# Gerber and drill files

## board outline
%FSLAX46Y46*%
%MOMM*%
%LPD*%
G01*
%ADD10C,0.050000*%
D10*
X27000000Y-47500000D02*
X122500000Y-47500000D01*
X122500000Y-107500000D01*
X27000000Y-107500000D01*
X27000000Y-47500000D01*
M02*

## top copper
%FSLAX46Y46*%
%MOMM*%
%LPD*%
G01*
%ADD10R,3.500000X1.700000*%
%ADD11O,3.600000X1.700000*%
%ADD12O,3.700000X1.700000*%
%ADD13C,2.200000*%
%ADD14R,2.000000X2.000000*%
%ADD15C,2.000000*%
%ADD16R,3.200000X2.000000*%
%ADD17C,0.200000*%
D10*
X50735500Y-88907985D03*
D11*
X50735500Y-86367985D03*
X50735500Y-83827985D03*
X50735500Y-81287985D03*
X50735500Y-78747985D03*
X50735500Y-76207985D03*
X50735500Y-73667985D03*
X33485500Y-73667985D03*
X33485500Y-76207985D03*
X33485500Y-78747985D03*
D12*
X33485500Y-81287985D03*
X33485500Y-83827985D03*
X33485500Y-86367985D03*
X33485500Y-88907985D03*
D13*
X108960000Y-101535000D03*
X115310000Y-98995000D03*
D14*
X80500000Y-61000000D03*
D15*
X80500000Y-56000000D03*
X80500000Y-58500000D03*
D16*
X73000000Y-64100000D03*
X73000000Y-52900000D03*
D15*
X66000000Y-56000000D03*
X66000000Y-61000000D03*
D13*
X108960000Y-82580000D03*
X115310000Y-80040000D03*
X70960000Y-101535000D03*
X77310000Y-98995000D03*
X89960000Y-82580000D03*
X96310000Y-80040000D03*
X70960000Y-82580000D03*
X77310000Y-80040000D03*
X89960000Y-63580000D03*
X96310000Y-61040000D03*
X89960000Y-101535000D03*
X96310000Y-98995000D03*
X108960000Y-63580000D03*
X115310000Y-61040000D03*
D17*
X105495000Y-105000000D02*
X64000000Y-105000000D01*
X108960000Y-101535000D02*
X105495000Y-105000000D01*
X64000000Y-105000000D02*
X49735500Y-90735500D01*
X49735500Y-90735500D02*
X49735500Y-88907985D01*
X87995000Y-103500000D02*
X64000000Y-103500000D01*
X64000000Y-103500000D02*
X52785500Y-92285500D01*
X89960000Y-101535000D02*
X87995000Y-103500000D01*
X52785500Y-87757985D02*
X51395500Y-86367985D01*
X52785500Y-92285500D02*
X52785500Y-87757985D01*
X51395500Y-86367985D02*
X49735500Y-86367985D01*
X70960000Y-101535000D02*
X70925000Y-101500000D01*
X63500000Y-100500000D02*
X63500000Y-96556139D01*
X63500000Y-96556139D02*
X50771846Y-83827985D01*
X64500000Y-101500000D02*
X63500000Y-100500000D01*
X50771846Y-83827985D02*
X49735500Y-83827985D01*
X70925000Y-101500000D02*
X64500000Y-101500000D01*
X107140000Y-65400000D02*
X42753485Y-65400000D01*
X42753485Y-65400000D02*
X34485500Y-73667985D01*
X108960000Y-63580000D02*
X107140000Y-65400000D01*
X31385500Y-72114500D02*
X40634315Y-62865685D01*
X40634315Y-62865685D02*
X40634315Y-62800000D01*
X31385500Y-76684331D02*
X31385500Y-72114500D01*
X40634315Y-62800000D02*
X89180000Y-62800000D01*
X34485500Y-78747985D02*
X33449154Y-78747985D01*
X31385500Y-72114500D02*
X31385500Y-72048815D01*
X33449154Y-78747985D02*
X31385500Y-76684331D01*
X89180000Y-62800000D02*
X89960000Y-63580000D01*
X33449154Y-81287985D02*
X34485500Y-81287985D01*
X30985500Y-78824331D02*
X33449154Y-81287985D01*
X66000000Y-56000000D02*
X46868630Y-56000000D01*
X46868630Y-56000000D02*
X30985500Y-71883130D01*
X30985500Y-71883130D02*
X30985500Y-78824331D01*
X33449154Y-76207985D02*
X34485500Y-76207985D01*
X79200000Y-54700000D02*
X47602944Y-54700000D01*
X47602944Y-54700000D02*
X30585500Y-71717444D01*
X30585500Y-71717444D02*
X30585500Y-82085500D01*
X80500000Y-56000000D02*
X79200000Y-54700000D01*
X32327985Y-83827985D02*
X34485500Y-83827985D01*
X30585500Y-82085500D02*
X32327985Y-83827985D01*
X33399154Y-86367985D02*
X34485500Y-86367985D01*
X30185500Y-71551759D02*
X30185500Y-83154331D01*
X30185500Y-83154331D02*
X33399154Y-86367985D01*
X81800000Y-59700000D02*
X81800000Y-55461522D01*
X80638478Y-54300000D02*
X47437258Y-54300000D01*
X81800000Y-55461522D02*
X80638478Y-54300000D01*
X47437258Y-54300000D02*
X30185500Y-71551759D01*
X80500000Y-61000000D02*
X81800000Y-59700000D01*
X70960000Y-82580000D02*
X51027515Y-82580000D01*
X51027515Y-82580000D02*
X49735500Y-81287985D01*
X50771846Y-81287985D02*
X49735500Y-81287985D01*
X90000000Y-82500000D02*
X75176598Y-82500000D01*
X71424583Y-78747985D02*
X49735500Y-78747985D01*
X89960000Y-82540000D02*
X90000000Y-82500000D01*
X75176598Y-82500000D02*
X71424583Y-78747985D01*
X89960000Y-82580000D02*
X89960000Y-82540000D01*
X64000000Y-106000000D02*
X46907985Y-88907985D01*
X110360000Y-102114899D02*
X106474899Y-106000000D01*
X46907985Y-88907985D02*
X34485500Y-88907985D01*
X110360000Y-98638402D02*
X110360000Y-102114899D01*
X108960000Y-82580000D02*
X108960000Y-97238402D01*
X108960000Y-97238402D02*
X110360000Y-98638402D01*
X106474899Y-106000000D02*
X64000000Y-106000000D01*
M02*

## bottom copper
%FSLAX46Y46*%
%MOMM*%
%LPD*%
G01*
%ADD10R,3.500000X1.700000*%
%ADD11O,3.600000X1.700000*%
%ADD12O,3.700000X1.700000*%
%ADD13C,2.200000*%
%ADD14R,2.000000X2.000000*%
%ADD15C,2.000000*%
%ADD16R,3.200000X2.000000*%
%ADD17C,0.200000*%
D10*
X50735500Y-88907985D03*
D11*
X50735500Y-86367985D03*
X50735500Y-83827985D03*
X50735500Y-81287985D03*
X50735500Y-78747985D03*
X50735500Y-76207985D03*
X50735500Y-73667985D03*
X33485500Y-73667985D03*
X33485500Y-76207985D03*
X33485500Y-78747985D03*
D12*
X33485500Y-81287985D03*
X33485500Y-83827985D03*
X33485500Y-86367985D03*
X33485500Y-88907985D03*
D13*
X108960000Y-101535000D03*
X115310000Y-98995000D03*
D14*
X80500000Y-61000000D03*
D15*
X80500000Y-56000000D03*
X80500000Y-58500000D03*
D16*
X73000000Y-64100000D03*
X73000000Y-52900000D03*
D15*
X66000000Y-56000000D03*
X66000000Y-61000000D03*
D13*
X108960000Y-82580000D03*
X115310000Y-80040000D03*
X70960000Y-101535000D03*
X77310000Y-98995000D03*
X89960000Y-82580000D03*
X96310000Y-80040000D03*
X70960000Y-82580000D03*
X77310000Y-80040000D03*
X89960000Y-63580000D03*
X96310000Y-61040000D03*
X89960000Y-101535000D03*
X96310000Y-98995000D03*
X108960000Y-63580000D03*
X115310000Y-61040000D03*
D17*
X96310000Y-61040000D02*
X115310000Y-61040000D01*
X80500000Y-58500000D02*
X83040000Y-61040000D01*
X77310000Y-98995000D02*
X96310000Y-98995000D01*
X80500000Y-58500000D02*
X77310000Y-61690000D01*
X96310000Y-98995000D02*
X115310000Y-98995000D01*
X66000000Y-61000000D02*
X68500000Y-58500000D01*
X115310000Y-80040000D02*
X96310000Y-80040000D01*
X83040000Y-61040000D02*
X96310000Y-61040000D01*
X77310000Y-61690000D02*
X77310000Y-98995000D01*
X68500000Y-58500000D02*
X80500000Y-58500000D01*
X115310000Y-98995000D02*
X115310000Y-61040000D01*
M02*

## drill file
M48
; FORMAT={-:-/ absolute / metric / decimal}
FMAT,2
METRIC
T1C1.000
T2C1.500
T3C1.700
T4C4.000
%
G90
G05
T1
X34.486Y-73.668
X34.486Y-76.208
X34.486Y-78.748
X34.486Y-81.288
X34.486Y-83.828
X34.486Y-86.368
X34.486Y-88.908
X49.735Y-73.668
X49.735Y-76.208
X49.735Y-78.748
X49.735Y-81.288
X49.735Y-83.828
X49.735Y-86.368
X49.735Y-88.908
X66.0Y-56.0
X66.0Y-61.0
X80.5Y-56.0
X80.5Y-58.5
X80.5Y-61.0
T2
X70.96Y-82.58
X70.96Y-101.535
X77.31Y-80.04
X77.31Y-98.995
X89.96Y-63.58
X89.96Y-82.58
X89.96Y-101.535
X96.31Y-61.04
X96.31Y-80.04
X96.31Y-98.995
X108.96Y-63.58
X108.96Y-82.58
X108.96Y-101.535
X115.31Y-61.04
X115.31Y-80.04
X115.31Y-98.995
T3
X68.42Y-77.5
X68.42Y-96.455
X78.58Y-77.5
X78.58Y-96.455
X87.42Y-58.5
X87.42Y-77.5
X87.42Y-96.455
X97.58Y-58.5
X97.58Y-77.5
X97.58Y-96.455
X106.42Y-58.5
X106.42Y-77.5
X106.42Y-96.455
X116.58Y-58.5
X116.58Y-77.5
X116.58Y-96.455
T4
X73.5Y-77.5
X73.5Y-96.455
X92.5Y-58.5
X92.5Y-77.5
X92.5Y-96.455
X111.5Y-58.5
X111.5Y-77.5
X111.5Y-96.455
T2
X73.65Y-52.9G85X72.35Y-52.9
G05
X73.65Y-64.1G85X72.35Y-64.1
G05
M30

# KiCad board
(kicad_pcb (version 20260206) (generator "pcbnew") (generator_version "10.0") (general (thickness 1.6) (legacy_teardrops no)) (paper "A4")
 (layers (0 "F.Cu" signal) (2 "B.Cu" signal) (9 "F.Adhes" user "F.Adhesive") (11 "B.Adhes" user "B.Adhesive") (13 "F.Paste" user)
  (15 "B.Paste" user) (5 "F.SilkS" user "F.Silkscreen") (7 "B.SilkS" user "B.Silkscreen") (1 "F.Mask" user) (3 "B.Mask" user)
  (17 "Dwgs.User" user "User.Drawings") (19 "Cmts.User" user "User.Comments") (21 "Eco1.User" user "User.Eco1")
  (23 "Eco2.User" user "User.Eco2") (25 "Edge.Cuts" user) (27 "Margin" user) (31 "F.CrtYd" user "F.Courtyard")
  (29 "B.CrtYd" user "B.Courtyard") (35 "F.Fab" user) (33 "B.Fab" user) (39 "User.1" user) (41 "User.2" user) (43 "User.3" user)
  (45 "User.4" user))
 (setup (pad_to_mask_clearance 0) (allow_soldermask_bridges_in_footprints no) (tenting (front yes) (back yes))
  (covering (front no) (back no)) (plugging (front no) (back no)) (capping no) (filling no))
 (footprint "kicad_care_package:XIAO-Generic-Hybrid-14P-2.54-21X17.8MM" (layer "F.Cu") (at 42.1105 81.287985 180)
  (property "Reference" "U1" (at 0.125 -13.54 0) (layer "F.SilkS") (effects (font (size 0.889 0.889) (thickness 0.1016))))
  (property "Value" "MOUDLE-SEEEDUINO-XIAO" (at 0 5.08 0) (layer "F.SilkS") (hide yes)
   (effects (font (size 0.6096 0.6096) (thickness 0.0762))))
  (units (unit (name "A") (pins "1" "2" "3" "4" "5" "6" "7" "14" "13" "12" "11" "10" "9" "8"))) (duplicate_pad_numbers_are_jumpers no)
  (pad "1" thru_hole rect (at -7.625 -7.62 180) (size 3.5 1.7) (drill 1 (offset -1 0)) (layers "*.Cu" "*.Mask") (remove_unused_layers no)
   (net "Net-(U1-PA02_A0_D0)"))
  (pad "2" thru_hole oval (at -7.625 -5.08 180) (size 3.6 1.7) (drill 1 (offset -1 0)) (layers "*.Cu" "*.Mask") (remove_unused_layers no)
   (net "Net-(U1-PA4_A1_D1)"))
  (pad "3" thru_hole oval (at -7.625 -2.54 180) (size 3.6 1.7) (drill 1 (offset -1 0)) (layers "*.Cu" "*.Mask") (remove_unused_layers no)
   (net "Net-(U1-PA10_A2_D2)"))
  (pad "4" thru_hole oval (at -7.625 0 180) (size 3.6 1.7) (drill 1 (offset -1 0)) (layers "*.Cu" "*.Mask") (remove_unused_layers no)
   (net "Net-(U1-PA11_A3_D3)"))
  (pad "5" thru_hole oval (at -7.625 2.54 180) (size 3.6 1.7) (drill 1 (offset -1 0)) (layers "*.Cu" "*.Mask") (remove_unused_layers no)
   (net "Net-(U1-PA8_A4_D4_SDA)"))
  (pad "6" thru_hole oval (at -7.625 5.08) (size 3.6 1.7) (drill 1 (offset 1 0)) (layers "*.Cu" "*.Mask") (remove_unused_layers no)
   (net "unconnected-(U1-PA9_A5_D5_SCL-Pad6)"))
  (pad "7" thru_hole oval (at -7.625 7.62 180) (size 3.6 1.7) (drill 1 (offset -1 0)) (layers "*.Cu" "*.Mask") (remove_unused_layers no)
   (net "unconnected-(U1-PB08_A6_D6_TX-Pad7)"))
  (pad "8" thru_hole oval (at 7.625 7.62 180) (size 3.6 1.7) (drill 1 (offset 1 0)) (layers "*.Cu" "*.Mask") (remove_unused_layers no)
   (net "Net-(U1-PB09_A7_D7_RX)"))
  (pad "9" thru_hole oval (at 7.625 5.08 180) (size 3.6 1.7) (drill 1 (offset 1 0)) (layers "*.Cu" "*.Mask") (remove_unused_layers no)
   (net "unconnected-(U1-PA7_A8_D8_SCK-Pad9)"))
  (pad "10" thru_hole oval (at 7.625 2.54 180) (size 3.6 1.7) (drill 1 (offset 1 0)) (layers "*.Cu" "*.Mask") (remove_unused_layers no)
   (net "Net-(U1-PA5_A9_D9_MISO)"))
  (pad "11" thru_hole oval (at 7.625 0 180) (size 3.7 1.7) (drill 1 (offset 1 0)) (layers "*.Cu" "*.Mask") (remove_unused_layers no)
   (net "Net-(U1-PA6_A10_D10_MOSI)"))
  (pad "12" thru_hole oval (at 7.625 -2.54 180) (size 3.7 1.7) (drill 1 (offset 1 0)) (layers "*.Cu" "*.Mask") (remove_unused_layers no)
   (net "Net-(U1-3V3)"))
  (pad "13" thru_hole oval (at 7.625 -5.08 180) (size 3.7 1.7) (drill 1 (offset 1 0)) (layers "*.Cu" "*.Mask") (remove_unused_layers no)
   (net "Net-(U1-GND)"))
  (pad "14" thru_hole oval (at 7.625 -7.62 180) (size 3.7 1.7) (drill 1 (offset 1 0)) (layers "*.Cu" "*.Mask") (remove_unused_layers no)
   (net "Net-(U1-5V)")))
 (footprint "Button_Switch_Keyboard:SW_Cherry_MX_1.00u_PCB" (layer "F.Cu") (at 108.96 101.535 180)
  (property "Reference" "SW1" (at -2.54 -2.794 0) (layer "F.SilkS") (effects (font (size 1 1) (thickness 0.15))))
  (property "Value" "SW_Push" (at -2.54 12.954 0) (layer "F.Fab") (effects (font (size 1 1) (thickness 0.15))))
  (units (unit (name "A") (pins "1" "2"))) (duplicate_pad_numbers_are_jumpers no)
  (pad "" np_thru_hole circle (at -7.62 5.08 180) (size 1.7 1.7) (drill 1.7) (layers "*.Cu" "*.Mask"))
  (pad "" np_thru_hole circle (at -2.54 5.08 180) (size 4 4) (drill 4) (layers "*.Cu" "*.Mask"))
  (pad "" np_thru_hole circle (at 2.54 5.08 180) (size 1.7 1.7) (drill 1.7) (layers "*.Cu" "*.Mask"))
  (pad "1" thru_hole circle (at 0 0 180) (size 2.2 2.2) (drill 1.5) (layers "*.Cu" "*.Mask") (remove_unused_layers no)
   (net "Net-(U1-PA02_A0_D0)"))
  (pad "2" thru_hole circle (at -6.35 2.54 180) (size 2.2 2.2) (drill 1.5) (layers "*.Cu" "*.Mask") (remove_unused_layers no) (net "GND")))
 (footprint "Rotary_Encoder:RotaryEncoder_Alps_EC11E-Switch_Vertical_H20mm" (layer "F.Cu") (at 80.5 61 180)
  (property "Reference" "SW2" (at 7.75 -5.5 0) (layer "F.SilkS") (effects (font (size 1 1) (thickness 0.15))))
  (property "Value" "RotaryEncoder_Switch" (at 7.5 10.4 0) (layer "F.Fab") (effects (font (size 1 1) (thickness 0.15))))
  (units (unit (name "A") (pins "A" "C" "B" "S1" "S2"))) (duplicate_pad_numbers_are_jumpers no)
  (pad "A" thru_hole rect (at 0 0 180) (size 2 2) (drill 1) (layers "*.Cu" "*.Mask") (remove_unused_layers no) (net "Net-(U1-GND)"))
  (pad "B" thru_hole circle (at 0 5 180) (size 2 2) (drill 1) (layers "*.Cu" "F.Mask") (remove_unused_layers no) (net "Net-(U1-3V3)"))
  (pad "C" thru_hole circle (at 0 2.5 180) (size 2 2) (drill 1) (layers "*.Cu" "*.Mask") (remove_unused_layers no) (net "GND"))
  (pad "MP" thru_hole rect (at 7.5 -3.1 180) (size 3.2 2) (drill oval 2.8 1.5) (layers "*.Cu" "*.Mask") (remove_unused_layers no))
  (pad "MP" thru_hole rect (at 7.5 8.1 180) (size 3.2 2) (drill oval 2.8 1.5) (layers "*.Cu" "*.Mask") (remove_unused_layers no))
  (pad "S1" thru_hole circle (at 14.5 5 180) (size 2 2) (drill 1) (layers "*.Cu" "*.Mask") (remove_unused_layers no)
   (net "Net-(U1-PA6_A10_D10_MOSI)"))
  (pad "S2" thru_hole circle (at 14.5 0 180) (size 2 2) (drill 1) (layers "*.Cu" "*.Mask") (remove_unused_layers no) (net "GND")))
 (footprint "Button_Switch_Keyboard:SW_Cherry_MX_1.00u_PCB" (layer "F.Cu") (at 108.96 82.58 180)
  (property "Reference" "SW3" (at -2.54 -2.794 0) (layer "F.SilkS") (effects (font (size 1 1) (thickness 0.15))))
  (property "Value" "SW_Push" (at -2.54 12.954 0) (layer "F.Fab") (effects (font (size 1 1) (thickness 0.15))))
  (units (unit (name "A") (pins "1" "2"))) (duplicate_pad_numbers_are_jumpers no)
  (pad "" np_thru_hole circle (at -7.62 5.08 180) (size 1.7 1.7) (drill 1.7) (layers "*.Cu" "*.Mask"))
  (pad "" np_thru_hole circle (at -2.54 5.08 180) (size 4 4) (drill 4) (layers "*.Cu" "*.Mask"))
  (pad "" np_thru_hole circle (at 2.54 5.08 180) (size 1.7 1.7) (drill 1.7) (layers "*.Cu" "*.Mask"))
  (pad "1" thru_hole circle (at 0 0 180) (size 2.2 2.2) (drill 1.5) (layers "*.Cu" "*.Mask") (remove_unused_layers no) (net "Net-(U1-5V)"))
  (pad "2" thru_hole circle (at -6.35 2.54 180) (size 2.2 2.2) (drill 1.5) (layers "*.Cu" "*.Mask") (remove_unused_layers no) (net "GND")))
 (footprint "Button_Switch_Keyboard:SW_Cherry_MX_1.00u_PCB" (layer "F.Cu") (at 70.96 101.535 180)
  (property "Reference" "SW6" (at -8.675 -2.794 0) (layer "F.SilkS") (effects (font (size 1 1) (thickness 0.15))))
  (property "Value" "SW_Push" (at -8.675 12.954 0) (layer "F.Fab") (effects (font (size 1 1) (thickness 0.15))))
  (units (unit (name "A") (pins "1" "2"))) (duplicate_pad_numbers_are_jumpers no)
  (pad "" np_thru_hole circle (at -7.62 5.08 180) (size 1.7 1.7) (drill 1.7) (layers "*.Cu" "*.Mask"))
  (pad "" np_thru_hole circle (at -2.54 5.08 180) (size 4 4) (drill 4) (layers "*.Cu" "*.Mask"))
  (pad "" np_thru_hole circle (at 2.54 5.08 180) (size 1.7 1.7) (drill 1.7) (layers "*.Cu" "*.Mask"))
  (pad "1" thru_hole circle (at 0 0 180) (size 2.2 2.2) (drill 1.5) (layers "*.Cu" "*.Mask") (remove_unused_layers no)
   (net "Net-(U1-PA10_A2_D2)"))
  (pad "2" thru_hole circle (at -6.35 2.54 180) (size 2.2 2.2) (drill 1.5) (layers "*.Cu" "*.Mask") (remove_unused_layers no) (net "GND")))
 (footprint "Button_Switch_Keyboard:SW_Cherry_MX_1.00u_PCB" (layer "F.Cu") (at 89.96 82.58 180)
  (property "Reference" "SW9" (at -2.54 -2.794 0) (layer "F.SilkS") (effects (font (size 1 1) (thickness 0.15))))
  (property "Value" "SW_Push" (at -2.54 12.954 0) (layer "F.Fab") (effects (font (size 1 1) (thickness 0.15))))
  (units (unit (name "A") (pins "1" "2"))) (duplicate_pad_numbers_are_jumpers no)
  (pad "" np_thru_hole circle (at -7.62 5.08 180) (size 1.7 1.7) (drill 1.7) (layers "*.Cu" "*.Mask"))
  (pad "" np_thru_hole circle (at -2.54 5.08 180) (size 4 4) (drill 4) (layers "*.Cu" "*.Mask"))
  (pad "" np_thru_hole circle (at 2.54 5.08 180) (size 1.7 1.7) (drill 1.7) (layers "*.Cu" "*.Mask"))
  (pad "1" thru_hole circle (at 0 0 180) (size 2.2 2.2) (drill 1.5) (layers "*.Cu" "*.Mask") (remove_unused_layers no)
   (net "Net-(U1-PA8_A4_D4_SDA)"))
  (pad "2" thru_hole circle (at -6.35 2.54 180) (size 2.2 2.2) (drill 1.5) (layers "*.Cu" "*.Mask") (remove_unused_layers no) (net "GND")))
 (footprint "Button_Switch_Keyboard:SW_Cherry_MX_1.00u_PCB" (layer "F.Cu") (at 70.96 82.58 180)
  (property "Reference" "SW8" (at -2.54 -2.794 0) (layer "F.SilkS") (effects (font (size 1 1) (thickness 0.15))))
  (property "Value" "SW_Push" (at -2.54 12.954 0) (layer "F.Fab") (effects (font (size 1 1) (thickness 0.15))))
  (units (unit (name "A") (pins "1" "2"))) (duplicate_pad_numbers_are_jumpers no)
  (pad "" np_thru_hole circle (at -7.62 5.08 180) (size 1.7 1.7) (drill 1.7) (layers "*.Cu" "*.Mask"))
  (pad "" np_thru_hole circle (at -2.54 5.08 180) (size 4 4) (drill 4) (layers "*.Cu" "*.Mask"))
  (pad "" np_thru_hole circle (at 2.54 5.08 180) (size 1.7 1.7) (drill 1.7) (layers "*.Cu" "*.Mask"))
  (pad "1" thru_hole circle (at 0 0 180) (size 2.2 2.2) (drill 1.5) (layers "*.Cu" "*.Mask") (remove_unused_layers no)
   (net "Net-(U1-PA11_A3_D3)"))
  (pad "2" thru_hole circle (at -6.35 2.54 180) (size 2.2 2.2) (drill 1.5) (layers "*.Cu" "*.Mask") (remove_unused_layers no) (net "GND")))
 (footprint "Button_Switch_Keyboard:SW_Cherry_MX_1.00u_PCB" (layer "F.Cu") (at 89.96 63.58 180)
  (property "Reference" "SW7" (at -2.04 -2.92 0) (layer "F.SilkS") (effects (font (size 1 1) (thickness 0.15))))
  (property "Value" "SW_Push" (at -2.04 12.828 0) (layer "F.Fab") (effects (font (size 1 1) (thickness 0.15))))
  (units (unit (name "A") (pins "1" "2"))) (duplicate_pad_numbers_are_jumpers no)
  (pad "" np_thru_hole circle (at -7.62 5.08 180) (size 1.7 1.7) (drill 1.7) (layers "*.Cu" "*.Mask"))
  (pad "" np_thru_hole circle (at -2.54 5.08 180) (size 4 4) (drill 4) (layers "*.Cu" "*.Mask"))
  (pad "" np_thru_hole circle (at 2.54 5.08 180) (size 1.7 1.7) (drill 1.7) (layers "*.Cu" "*.Mask"))
  (pad "1" thru_hole circle (at 0 0 180) (size 2.2 2.2) (drill 1.5) (layers "*.Cu" "*.Mask") (remove_unused_layers no)
   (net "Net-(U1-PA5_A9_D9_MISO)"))
  (pad "2" thru_hole circle (at -6.35 2.54 180) (size 2.2 2.2) (drill 1.5) (layers "*.Cu" "*.Mask") (remove_unused_layers no) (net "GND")))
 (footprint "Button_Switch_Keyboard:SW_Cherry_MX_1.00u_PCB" (layer "F.Cu") (at 89.96 101.535 180)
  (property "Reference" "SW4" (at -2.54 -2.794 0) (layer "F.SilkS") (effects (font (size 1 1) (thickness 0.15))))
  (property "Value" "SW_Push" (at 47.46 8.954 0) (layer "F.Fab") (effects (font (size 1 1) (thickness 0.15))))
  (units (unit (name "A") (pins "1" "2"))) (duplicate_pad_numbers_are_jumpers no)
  (pad "" np_thru_hole circle (at -7.62 5.08 180) (size 1.7 1.7) (drill 1.7) (layers "*.Cu" "*.Mask"))
  (pad "" np_thru_hole circle (at -2.54 5.08 180) (size 4 4) (drill 4) (layers "*.Cu" "*.Mask"))
  (pad "" np_thru_hole circle (at 2.54 5.08 180) (size 1.7 1.7) (drill 1.7) (layers "*.Cu" "*.Mask"))
  (pad "1" thru_hole circle (at 0 0 180) (size 2.2 2.2) (drill 1.5) (layers "*.Cu" "*.Mask") (remove_unused_layers no)
   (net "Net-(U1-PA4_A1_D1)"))
  (pad "2" thru_hole circle (at -6.35 2.54 180) (size 2.2 2.2) (drill 1.5) (layers "*.Cu" "*.Mask") (remove_unused_layers no) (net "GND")))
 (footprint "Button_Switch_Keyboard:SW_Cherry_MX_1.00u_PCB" (layer "F.Cu") (at 108.96 63.58 180)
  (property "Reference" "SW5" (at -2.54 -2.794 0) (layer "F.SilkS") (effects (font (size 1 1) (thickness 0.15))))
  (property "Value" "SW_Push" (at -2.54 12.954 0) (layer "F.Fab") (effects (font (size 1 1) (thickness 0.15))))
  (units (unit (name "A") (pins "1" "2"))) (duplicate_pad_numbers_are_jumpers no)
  (pad "" np_thru_hole circle (at -7.62 5.08 180) (size 1.7 1.7) (drill 1.7) (layers "*.Cu" "*.Mask"))
  (pad "" np_thru_hole circle (at -2.54 5.08 180) (size 4 4) (drill 4) (layers "*.Cu" "*.Mask"))
  (pad "" np_thru_hole circle (at 2.54 5.08 180) (size 1.7 1.7) (drill 1.7) (layers "*.Cu" "*.Mask"))
  (pad "1" thru_hole circle (at 0 0 180) (size 2.2 2.2) (drill 1.5) (layers "*.Cu" "*.Mask") (remove_unused_layers no)
   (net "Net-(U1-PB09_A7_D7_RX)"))
  (pad "2" thru_hole circle (at -6.35 2.54 180) (size 2.2 2.2) (drill 1.5) (layers "*.Cu" "*.Mask") (remove_unused_layers no) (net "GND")))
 (gr_rect (start 27 47.5) (end 122.5 107.5) (stroke (width 0.05) (type default)) (fill no) (layer "Edge.Cuts"))
 (segment (start 105.495 105) (end 64 105) (width 0.2) (layer "F.Cu") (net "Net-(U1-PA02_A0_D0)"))
 (segment (start 108.96 101.535) (end 105.495 105) (width 0.2) (layer "F.Cu") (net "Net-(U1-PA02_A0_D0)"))
 (segment (start 64 105) (end 49.7355 90.7355) (width 0.2) (layer "F.Cu") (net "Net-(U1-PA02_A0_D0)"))
 (segment (start 49.7355 90.7355) (end 49.7355 88.907985) (width 0.2) (layer "F.Cu") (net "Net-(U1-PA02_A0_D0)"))
 (segment (start 87.995 103.5) (end 64 103.5) (width 0.2) (layer "F.Cu") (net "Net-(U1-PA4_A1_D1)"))
 (segment (start 64 103.5) (end 52.7855 92.2855) (width 0.2) (layer "F.Cu") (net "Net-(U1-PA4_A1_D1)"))
 (segment (start 89.96 101.535) (end 87.995 103.5) (width 0.2) (layer "F.Cu") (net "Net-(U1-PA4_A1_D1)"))
 (segment (start 52.7855 87.757985) (end 51.3955 86.367985) (width 0.2) (layer "F.Cu") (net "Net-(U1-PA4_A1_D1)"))
 (segment (start 52.7855 92.2855) (end 52.7855 87.757985) (width 0.2) (layer "F.Cu") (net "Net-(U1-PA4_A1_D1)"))
 (segment (start 51.3955 86.367985) (end 49.7355 86.367985) (width 0.2) (layer "F.Cu") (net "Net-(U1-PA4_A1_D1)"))
 (segment (start 70.96 101.535) (end 70.925 101.5) (width 0.2) (layer "F.Cu") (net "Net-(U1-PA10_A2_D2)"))
 (segment (start 63.5 100.5) (end 63.5 96.556139) (width 0.2) (layer "F.Cu") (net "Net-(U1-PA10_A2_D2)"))
 (segment (start 63.5 96.556139) (end 50.771846 83.827985) (width 0.2) (layer "F.Cu") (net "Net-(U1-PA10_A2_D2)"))
 (segment (start 64.5 101.5) (end 63.5 100.5) (width 0.2) (layer "F.Cu") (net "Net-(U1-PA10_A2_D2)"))
 (segment (start 50.771846 83.827985) (end 49.7355 83.827985) (width 0.2) (layer "F.Cu") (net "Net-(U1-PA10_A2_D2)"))
 (segment (start 70.925 101.5) (end 64.5 101.5) (width 0.2) (layer "F.Cu") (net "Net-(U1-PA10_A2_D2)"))
 (segment (start 107.14 65.4) (end 42.753485 65.4) (width 0.2) (layer "F.Cu") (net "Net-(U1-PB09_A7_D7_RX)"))
 (segment (start 42.753485 65.4) (end 34.4855 73.667985) (width 0.2) (layer "F.Cu") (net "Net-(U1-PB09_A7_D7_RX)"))
 (segment (start 108.96 63.58) (end 107.14 65.4) (width 0.2) (layer "F.Cu") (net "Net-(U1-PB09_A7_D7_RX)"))
 (segment (start 31.3855 72.1145) (end 40.634315 62.865685) (width 0.2) (layer "F.Cu") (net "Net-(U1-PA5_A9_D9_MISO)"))
 (segment (start 40.634315 62.865685) (end 40.634315 62.8) (width 0.2) (layer "F.Cu") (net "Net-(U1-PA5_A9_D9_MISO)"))
 (segment (start 31.3855 76.684331) (end 31.3855 72.1145) (width 0.2) (layer "F.Cu") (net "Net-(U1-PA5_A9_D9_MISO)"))
 (segment (start 40.634315 62.8) (end 89.18 62.8) (width 0.2) (layer "F.Cu") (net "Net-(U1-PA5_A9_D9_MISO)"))
 (segment (start 34.4855 78.747985) (end 33.449154 78.747985) (width 0.2) (layer "F.Cu") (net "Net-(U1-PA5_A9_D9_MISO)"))
 (segment (start 31.3855 72.1145) (end 31.3855 72.048815) (width 0.2) (layer "F.Cu") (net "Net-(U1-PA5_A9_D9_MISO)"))
 (segment (start 33.449154 78.747985) (end 31.3855 76.684331) (width 0.2) (layer "F.Cu") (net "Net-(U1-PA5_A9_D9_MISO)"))
 (segment (start 89.18 62.8) (end 89.96 63.58) (width 0.2) (layer "F.Cu") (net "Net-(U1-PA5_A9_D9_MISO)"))
 (segment (start 33.449154 81.287985) (end 34.4855 81.287985) (width 0.2) (layer "F.Cu") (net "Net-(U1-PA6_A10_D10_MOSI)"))
 (segment (start 30.9855 78.824331) (end 33.449154 81.287985) (width 0.2) (layer "F.Cu") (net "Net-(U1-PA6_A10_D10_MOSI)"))
 (segment (start 66 56) (end 46.86863 56) (width 0.2) (layer "F.Cu") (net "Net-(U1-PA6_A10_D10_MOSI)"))
 (segment (start 46.86863 56) (end 30.9855 71.88313) (width 0.2) (layer "F.Cu") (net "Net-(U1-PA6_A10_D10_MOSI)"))
 (segment (start 30.9855 71.88313) (end 30.9855 78.824331) (width 0.2) (layer "F.Cu") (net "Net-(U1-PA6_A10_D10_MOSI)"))
 (segment (start 96.31 61.04) (end 115.31 61.04) (width 0.2) (layer "B.Cu") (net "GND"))
 (segment (start 80.5 58.5) (end 83.04 61.04) (width 0.2) (layer "B.Cu") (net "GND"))
 (segment (start 77.31 98.995) (end 96.31 98.995) (width 0.2) (layer "B.Cu") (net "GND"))
 (segment (start 80.5 58.5) (end 77.31 61.69) (width 0.2) (layer "B.Cu") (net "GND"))
 (segment (start 96.31 98.995) (end 115.31 98.995) (width 0.2) (layer "B.Cu") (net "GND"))
 (segment (start 66 61) (end 68.5 58.5) (width 0.2) (layer "B.Cu") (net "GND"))
 (segment (start 115.31 80.04) (end 96.31 80.04) (width 0.2) (layer "B.Cu") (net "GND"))
 (segment (start 83.04 61.04) (end 96.31 61.04) (width 0.2) (layer "B.Cu") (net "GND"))
 (segment (start 77.31 61.69) (end 77.31 98.995) (width 0.2) (layer "B.Cu") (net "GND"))
 (segment (start 68.5 58.5) (end 80.5 58.5) (width 0.2) (layer "B.Cu") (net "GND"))
 (segment (start 115.31 98.995) (end 115.31 61.04) (width 0.2) (layer "B.Cu") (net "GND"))
 (segment (start 33.449154 76.207985) (end 34.4855 76.207985) (width 0.2) (layer "F.Cu") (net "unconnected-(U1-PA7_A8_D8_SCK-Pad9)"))
 (segment (start 79.2 54.7) (end 47.602944 54.7) (width 0.2) (layer "F.Cu") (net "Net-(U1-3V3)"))
 (segment (start 47.602944 54.7) (end 30.5855 71.717444) (width 0.2) (layer "F.Cu") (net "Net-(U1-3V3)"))
 (segment (start 30.5855 71.717444) (end 30.5855 82.0855) (width 0.2) (layer "F.Cu") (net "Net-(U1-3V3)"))
 (segment (start 80.5 56) (end 79.2 54.7) (width 0.2) (layer "F.Cu") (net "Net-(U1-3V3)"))
 (segment (start 32.327985 83.827985) (end 34.4855 83.827985) (width 0.2) (layer "F.Cu") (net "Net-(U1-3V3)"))
 (segment (start 30.5855 82.0855) (end 32.327985 83.827985) (width 0.2) (layer "F.Cu") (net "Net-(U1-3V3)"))
 (segment (start 33.399154 86.367985) (end 34.4855 86.367985) (width 0.2) (layer "F.Cu") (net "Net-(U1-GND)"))
 (segment (start 30.1855 71.551759) (end 30.1855 83.154331) (width 0.2) (layer "F.Cu") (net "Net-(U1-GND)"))
 (segment (start 30.1855 83.154331) (end 33.399154 86.367985) (width 0.2) (layer "F.Cu") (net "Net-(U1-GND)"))
 (segment (start 81.8 59.7) (end 81.8 55.461522) (width 0.2) (layer "F.Cu") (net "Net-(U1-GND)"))
 (segment (start 80.638478 54.3) (end 47.437258 54.3) (width 0.2) (layer "F.Cu") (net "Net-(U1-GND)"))
 (segment (start 81.8 55.461522) (end 80.638478 54.3) (width 0.2) (layer "F.Cu") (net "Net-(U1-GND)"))
 (segment (start 47.437258 54.3) (end 30.1855 71.551759) (width 0.2) (layer "F.Cu") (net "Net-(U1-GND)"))
 (segment (start 80.5 61) (end 81.8 59.7) (width 0.2) (layer "F.Cu") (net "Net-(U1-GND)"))
 (segment (start 70.96 82.58) (end 51.027515 82.58) (width 0.2) (layer "F.Cu") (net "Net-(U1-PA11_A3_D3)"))
 (segment (start 51.027515 82.58) (end 49.7355 81.287985) (width 0.2) (layer "F.Cu") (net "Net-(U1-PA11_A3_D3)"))
 (segment (start 50.771846 81.287985) (end 49.7355 81.287985) (width 0.2) (layer "F.Cu") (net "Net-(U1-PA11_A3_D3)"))
 (segment (start 90 82.5) (end 75.176598 82.5) (width 0.2) (layer "F.Cu") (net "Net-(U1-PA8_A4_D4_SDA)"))
 (segment (start 71.424583 78.747985) (end 49.7355 78.747985) (width 0.2) (layer "F.Cu") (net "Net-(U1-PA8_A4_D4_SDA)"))
 (segment (start 89.96 82.54) (end 90 82.5) (width 0.2) (layer "F.Cu") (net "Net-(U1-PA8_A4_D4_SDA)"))
 (segment (start 75.176598 82.5) (end 71.424583 78.747985) (width 0.2) (layer "F.Cu") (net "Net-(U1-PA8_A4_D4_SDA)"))
 (segment (start 89.96 82.58) (end 89.96 82.54) (width 0.2) (layer "F.Cu") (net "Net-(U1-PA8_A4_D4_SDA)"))
 (segment (start 64 106) (end 46.907985 88.907985) (width 0.2) (layer "F.Cu") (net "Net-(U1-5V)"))
 (segment (start 110.36 102.114899) (end 106.474899 106) (width 0.2) (layer "F.Cu") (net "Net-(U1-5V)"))
 (segment (start 46.907985 88.907985) (end 34.4855 88.907985) (width 0.2) (layer "F.Cu") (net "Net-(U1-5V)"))
 (segment (start 110.36 98.638402) (end 110.36 102.114899) (width 0.2) (layer "F.Cu") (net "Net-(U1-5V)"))
 (segment (start 108.96 82.58) (end 108.96 97.238402) (width 0.2) (layer "F.Cu") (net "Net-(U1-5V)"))
 (segment (start 108.96 97.238402) (end 110.36 98.638402) (width 0.2) (layer "F.Cu") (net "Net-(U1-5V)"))
 (segment (start 106.474899 106) (end 64 106) (width 0.2) (layer "F.Cu") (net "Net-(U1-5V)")))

